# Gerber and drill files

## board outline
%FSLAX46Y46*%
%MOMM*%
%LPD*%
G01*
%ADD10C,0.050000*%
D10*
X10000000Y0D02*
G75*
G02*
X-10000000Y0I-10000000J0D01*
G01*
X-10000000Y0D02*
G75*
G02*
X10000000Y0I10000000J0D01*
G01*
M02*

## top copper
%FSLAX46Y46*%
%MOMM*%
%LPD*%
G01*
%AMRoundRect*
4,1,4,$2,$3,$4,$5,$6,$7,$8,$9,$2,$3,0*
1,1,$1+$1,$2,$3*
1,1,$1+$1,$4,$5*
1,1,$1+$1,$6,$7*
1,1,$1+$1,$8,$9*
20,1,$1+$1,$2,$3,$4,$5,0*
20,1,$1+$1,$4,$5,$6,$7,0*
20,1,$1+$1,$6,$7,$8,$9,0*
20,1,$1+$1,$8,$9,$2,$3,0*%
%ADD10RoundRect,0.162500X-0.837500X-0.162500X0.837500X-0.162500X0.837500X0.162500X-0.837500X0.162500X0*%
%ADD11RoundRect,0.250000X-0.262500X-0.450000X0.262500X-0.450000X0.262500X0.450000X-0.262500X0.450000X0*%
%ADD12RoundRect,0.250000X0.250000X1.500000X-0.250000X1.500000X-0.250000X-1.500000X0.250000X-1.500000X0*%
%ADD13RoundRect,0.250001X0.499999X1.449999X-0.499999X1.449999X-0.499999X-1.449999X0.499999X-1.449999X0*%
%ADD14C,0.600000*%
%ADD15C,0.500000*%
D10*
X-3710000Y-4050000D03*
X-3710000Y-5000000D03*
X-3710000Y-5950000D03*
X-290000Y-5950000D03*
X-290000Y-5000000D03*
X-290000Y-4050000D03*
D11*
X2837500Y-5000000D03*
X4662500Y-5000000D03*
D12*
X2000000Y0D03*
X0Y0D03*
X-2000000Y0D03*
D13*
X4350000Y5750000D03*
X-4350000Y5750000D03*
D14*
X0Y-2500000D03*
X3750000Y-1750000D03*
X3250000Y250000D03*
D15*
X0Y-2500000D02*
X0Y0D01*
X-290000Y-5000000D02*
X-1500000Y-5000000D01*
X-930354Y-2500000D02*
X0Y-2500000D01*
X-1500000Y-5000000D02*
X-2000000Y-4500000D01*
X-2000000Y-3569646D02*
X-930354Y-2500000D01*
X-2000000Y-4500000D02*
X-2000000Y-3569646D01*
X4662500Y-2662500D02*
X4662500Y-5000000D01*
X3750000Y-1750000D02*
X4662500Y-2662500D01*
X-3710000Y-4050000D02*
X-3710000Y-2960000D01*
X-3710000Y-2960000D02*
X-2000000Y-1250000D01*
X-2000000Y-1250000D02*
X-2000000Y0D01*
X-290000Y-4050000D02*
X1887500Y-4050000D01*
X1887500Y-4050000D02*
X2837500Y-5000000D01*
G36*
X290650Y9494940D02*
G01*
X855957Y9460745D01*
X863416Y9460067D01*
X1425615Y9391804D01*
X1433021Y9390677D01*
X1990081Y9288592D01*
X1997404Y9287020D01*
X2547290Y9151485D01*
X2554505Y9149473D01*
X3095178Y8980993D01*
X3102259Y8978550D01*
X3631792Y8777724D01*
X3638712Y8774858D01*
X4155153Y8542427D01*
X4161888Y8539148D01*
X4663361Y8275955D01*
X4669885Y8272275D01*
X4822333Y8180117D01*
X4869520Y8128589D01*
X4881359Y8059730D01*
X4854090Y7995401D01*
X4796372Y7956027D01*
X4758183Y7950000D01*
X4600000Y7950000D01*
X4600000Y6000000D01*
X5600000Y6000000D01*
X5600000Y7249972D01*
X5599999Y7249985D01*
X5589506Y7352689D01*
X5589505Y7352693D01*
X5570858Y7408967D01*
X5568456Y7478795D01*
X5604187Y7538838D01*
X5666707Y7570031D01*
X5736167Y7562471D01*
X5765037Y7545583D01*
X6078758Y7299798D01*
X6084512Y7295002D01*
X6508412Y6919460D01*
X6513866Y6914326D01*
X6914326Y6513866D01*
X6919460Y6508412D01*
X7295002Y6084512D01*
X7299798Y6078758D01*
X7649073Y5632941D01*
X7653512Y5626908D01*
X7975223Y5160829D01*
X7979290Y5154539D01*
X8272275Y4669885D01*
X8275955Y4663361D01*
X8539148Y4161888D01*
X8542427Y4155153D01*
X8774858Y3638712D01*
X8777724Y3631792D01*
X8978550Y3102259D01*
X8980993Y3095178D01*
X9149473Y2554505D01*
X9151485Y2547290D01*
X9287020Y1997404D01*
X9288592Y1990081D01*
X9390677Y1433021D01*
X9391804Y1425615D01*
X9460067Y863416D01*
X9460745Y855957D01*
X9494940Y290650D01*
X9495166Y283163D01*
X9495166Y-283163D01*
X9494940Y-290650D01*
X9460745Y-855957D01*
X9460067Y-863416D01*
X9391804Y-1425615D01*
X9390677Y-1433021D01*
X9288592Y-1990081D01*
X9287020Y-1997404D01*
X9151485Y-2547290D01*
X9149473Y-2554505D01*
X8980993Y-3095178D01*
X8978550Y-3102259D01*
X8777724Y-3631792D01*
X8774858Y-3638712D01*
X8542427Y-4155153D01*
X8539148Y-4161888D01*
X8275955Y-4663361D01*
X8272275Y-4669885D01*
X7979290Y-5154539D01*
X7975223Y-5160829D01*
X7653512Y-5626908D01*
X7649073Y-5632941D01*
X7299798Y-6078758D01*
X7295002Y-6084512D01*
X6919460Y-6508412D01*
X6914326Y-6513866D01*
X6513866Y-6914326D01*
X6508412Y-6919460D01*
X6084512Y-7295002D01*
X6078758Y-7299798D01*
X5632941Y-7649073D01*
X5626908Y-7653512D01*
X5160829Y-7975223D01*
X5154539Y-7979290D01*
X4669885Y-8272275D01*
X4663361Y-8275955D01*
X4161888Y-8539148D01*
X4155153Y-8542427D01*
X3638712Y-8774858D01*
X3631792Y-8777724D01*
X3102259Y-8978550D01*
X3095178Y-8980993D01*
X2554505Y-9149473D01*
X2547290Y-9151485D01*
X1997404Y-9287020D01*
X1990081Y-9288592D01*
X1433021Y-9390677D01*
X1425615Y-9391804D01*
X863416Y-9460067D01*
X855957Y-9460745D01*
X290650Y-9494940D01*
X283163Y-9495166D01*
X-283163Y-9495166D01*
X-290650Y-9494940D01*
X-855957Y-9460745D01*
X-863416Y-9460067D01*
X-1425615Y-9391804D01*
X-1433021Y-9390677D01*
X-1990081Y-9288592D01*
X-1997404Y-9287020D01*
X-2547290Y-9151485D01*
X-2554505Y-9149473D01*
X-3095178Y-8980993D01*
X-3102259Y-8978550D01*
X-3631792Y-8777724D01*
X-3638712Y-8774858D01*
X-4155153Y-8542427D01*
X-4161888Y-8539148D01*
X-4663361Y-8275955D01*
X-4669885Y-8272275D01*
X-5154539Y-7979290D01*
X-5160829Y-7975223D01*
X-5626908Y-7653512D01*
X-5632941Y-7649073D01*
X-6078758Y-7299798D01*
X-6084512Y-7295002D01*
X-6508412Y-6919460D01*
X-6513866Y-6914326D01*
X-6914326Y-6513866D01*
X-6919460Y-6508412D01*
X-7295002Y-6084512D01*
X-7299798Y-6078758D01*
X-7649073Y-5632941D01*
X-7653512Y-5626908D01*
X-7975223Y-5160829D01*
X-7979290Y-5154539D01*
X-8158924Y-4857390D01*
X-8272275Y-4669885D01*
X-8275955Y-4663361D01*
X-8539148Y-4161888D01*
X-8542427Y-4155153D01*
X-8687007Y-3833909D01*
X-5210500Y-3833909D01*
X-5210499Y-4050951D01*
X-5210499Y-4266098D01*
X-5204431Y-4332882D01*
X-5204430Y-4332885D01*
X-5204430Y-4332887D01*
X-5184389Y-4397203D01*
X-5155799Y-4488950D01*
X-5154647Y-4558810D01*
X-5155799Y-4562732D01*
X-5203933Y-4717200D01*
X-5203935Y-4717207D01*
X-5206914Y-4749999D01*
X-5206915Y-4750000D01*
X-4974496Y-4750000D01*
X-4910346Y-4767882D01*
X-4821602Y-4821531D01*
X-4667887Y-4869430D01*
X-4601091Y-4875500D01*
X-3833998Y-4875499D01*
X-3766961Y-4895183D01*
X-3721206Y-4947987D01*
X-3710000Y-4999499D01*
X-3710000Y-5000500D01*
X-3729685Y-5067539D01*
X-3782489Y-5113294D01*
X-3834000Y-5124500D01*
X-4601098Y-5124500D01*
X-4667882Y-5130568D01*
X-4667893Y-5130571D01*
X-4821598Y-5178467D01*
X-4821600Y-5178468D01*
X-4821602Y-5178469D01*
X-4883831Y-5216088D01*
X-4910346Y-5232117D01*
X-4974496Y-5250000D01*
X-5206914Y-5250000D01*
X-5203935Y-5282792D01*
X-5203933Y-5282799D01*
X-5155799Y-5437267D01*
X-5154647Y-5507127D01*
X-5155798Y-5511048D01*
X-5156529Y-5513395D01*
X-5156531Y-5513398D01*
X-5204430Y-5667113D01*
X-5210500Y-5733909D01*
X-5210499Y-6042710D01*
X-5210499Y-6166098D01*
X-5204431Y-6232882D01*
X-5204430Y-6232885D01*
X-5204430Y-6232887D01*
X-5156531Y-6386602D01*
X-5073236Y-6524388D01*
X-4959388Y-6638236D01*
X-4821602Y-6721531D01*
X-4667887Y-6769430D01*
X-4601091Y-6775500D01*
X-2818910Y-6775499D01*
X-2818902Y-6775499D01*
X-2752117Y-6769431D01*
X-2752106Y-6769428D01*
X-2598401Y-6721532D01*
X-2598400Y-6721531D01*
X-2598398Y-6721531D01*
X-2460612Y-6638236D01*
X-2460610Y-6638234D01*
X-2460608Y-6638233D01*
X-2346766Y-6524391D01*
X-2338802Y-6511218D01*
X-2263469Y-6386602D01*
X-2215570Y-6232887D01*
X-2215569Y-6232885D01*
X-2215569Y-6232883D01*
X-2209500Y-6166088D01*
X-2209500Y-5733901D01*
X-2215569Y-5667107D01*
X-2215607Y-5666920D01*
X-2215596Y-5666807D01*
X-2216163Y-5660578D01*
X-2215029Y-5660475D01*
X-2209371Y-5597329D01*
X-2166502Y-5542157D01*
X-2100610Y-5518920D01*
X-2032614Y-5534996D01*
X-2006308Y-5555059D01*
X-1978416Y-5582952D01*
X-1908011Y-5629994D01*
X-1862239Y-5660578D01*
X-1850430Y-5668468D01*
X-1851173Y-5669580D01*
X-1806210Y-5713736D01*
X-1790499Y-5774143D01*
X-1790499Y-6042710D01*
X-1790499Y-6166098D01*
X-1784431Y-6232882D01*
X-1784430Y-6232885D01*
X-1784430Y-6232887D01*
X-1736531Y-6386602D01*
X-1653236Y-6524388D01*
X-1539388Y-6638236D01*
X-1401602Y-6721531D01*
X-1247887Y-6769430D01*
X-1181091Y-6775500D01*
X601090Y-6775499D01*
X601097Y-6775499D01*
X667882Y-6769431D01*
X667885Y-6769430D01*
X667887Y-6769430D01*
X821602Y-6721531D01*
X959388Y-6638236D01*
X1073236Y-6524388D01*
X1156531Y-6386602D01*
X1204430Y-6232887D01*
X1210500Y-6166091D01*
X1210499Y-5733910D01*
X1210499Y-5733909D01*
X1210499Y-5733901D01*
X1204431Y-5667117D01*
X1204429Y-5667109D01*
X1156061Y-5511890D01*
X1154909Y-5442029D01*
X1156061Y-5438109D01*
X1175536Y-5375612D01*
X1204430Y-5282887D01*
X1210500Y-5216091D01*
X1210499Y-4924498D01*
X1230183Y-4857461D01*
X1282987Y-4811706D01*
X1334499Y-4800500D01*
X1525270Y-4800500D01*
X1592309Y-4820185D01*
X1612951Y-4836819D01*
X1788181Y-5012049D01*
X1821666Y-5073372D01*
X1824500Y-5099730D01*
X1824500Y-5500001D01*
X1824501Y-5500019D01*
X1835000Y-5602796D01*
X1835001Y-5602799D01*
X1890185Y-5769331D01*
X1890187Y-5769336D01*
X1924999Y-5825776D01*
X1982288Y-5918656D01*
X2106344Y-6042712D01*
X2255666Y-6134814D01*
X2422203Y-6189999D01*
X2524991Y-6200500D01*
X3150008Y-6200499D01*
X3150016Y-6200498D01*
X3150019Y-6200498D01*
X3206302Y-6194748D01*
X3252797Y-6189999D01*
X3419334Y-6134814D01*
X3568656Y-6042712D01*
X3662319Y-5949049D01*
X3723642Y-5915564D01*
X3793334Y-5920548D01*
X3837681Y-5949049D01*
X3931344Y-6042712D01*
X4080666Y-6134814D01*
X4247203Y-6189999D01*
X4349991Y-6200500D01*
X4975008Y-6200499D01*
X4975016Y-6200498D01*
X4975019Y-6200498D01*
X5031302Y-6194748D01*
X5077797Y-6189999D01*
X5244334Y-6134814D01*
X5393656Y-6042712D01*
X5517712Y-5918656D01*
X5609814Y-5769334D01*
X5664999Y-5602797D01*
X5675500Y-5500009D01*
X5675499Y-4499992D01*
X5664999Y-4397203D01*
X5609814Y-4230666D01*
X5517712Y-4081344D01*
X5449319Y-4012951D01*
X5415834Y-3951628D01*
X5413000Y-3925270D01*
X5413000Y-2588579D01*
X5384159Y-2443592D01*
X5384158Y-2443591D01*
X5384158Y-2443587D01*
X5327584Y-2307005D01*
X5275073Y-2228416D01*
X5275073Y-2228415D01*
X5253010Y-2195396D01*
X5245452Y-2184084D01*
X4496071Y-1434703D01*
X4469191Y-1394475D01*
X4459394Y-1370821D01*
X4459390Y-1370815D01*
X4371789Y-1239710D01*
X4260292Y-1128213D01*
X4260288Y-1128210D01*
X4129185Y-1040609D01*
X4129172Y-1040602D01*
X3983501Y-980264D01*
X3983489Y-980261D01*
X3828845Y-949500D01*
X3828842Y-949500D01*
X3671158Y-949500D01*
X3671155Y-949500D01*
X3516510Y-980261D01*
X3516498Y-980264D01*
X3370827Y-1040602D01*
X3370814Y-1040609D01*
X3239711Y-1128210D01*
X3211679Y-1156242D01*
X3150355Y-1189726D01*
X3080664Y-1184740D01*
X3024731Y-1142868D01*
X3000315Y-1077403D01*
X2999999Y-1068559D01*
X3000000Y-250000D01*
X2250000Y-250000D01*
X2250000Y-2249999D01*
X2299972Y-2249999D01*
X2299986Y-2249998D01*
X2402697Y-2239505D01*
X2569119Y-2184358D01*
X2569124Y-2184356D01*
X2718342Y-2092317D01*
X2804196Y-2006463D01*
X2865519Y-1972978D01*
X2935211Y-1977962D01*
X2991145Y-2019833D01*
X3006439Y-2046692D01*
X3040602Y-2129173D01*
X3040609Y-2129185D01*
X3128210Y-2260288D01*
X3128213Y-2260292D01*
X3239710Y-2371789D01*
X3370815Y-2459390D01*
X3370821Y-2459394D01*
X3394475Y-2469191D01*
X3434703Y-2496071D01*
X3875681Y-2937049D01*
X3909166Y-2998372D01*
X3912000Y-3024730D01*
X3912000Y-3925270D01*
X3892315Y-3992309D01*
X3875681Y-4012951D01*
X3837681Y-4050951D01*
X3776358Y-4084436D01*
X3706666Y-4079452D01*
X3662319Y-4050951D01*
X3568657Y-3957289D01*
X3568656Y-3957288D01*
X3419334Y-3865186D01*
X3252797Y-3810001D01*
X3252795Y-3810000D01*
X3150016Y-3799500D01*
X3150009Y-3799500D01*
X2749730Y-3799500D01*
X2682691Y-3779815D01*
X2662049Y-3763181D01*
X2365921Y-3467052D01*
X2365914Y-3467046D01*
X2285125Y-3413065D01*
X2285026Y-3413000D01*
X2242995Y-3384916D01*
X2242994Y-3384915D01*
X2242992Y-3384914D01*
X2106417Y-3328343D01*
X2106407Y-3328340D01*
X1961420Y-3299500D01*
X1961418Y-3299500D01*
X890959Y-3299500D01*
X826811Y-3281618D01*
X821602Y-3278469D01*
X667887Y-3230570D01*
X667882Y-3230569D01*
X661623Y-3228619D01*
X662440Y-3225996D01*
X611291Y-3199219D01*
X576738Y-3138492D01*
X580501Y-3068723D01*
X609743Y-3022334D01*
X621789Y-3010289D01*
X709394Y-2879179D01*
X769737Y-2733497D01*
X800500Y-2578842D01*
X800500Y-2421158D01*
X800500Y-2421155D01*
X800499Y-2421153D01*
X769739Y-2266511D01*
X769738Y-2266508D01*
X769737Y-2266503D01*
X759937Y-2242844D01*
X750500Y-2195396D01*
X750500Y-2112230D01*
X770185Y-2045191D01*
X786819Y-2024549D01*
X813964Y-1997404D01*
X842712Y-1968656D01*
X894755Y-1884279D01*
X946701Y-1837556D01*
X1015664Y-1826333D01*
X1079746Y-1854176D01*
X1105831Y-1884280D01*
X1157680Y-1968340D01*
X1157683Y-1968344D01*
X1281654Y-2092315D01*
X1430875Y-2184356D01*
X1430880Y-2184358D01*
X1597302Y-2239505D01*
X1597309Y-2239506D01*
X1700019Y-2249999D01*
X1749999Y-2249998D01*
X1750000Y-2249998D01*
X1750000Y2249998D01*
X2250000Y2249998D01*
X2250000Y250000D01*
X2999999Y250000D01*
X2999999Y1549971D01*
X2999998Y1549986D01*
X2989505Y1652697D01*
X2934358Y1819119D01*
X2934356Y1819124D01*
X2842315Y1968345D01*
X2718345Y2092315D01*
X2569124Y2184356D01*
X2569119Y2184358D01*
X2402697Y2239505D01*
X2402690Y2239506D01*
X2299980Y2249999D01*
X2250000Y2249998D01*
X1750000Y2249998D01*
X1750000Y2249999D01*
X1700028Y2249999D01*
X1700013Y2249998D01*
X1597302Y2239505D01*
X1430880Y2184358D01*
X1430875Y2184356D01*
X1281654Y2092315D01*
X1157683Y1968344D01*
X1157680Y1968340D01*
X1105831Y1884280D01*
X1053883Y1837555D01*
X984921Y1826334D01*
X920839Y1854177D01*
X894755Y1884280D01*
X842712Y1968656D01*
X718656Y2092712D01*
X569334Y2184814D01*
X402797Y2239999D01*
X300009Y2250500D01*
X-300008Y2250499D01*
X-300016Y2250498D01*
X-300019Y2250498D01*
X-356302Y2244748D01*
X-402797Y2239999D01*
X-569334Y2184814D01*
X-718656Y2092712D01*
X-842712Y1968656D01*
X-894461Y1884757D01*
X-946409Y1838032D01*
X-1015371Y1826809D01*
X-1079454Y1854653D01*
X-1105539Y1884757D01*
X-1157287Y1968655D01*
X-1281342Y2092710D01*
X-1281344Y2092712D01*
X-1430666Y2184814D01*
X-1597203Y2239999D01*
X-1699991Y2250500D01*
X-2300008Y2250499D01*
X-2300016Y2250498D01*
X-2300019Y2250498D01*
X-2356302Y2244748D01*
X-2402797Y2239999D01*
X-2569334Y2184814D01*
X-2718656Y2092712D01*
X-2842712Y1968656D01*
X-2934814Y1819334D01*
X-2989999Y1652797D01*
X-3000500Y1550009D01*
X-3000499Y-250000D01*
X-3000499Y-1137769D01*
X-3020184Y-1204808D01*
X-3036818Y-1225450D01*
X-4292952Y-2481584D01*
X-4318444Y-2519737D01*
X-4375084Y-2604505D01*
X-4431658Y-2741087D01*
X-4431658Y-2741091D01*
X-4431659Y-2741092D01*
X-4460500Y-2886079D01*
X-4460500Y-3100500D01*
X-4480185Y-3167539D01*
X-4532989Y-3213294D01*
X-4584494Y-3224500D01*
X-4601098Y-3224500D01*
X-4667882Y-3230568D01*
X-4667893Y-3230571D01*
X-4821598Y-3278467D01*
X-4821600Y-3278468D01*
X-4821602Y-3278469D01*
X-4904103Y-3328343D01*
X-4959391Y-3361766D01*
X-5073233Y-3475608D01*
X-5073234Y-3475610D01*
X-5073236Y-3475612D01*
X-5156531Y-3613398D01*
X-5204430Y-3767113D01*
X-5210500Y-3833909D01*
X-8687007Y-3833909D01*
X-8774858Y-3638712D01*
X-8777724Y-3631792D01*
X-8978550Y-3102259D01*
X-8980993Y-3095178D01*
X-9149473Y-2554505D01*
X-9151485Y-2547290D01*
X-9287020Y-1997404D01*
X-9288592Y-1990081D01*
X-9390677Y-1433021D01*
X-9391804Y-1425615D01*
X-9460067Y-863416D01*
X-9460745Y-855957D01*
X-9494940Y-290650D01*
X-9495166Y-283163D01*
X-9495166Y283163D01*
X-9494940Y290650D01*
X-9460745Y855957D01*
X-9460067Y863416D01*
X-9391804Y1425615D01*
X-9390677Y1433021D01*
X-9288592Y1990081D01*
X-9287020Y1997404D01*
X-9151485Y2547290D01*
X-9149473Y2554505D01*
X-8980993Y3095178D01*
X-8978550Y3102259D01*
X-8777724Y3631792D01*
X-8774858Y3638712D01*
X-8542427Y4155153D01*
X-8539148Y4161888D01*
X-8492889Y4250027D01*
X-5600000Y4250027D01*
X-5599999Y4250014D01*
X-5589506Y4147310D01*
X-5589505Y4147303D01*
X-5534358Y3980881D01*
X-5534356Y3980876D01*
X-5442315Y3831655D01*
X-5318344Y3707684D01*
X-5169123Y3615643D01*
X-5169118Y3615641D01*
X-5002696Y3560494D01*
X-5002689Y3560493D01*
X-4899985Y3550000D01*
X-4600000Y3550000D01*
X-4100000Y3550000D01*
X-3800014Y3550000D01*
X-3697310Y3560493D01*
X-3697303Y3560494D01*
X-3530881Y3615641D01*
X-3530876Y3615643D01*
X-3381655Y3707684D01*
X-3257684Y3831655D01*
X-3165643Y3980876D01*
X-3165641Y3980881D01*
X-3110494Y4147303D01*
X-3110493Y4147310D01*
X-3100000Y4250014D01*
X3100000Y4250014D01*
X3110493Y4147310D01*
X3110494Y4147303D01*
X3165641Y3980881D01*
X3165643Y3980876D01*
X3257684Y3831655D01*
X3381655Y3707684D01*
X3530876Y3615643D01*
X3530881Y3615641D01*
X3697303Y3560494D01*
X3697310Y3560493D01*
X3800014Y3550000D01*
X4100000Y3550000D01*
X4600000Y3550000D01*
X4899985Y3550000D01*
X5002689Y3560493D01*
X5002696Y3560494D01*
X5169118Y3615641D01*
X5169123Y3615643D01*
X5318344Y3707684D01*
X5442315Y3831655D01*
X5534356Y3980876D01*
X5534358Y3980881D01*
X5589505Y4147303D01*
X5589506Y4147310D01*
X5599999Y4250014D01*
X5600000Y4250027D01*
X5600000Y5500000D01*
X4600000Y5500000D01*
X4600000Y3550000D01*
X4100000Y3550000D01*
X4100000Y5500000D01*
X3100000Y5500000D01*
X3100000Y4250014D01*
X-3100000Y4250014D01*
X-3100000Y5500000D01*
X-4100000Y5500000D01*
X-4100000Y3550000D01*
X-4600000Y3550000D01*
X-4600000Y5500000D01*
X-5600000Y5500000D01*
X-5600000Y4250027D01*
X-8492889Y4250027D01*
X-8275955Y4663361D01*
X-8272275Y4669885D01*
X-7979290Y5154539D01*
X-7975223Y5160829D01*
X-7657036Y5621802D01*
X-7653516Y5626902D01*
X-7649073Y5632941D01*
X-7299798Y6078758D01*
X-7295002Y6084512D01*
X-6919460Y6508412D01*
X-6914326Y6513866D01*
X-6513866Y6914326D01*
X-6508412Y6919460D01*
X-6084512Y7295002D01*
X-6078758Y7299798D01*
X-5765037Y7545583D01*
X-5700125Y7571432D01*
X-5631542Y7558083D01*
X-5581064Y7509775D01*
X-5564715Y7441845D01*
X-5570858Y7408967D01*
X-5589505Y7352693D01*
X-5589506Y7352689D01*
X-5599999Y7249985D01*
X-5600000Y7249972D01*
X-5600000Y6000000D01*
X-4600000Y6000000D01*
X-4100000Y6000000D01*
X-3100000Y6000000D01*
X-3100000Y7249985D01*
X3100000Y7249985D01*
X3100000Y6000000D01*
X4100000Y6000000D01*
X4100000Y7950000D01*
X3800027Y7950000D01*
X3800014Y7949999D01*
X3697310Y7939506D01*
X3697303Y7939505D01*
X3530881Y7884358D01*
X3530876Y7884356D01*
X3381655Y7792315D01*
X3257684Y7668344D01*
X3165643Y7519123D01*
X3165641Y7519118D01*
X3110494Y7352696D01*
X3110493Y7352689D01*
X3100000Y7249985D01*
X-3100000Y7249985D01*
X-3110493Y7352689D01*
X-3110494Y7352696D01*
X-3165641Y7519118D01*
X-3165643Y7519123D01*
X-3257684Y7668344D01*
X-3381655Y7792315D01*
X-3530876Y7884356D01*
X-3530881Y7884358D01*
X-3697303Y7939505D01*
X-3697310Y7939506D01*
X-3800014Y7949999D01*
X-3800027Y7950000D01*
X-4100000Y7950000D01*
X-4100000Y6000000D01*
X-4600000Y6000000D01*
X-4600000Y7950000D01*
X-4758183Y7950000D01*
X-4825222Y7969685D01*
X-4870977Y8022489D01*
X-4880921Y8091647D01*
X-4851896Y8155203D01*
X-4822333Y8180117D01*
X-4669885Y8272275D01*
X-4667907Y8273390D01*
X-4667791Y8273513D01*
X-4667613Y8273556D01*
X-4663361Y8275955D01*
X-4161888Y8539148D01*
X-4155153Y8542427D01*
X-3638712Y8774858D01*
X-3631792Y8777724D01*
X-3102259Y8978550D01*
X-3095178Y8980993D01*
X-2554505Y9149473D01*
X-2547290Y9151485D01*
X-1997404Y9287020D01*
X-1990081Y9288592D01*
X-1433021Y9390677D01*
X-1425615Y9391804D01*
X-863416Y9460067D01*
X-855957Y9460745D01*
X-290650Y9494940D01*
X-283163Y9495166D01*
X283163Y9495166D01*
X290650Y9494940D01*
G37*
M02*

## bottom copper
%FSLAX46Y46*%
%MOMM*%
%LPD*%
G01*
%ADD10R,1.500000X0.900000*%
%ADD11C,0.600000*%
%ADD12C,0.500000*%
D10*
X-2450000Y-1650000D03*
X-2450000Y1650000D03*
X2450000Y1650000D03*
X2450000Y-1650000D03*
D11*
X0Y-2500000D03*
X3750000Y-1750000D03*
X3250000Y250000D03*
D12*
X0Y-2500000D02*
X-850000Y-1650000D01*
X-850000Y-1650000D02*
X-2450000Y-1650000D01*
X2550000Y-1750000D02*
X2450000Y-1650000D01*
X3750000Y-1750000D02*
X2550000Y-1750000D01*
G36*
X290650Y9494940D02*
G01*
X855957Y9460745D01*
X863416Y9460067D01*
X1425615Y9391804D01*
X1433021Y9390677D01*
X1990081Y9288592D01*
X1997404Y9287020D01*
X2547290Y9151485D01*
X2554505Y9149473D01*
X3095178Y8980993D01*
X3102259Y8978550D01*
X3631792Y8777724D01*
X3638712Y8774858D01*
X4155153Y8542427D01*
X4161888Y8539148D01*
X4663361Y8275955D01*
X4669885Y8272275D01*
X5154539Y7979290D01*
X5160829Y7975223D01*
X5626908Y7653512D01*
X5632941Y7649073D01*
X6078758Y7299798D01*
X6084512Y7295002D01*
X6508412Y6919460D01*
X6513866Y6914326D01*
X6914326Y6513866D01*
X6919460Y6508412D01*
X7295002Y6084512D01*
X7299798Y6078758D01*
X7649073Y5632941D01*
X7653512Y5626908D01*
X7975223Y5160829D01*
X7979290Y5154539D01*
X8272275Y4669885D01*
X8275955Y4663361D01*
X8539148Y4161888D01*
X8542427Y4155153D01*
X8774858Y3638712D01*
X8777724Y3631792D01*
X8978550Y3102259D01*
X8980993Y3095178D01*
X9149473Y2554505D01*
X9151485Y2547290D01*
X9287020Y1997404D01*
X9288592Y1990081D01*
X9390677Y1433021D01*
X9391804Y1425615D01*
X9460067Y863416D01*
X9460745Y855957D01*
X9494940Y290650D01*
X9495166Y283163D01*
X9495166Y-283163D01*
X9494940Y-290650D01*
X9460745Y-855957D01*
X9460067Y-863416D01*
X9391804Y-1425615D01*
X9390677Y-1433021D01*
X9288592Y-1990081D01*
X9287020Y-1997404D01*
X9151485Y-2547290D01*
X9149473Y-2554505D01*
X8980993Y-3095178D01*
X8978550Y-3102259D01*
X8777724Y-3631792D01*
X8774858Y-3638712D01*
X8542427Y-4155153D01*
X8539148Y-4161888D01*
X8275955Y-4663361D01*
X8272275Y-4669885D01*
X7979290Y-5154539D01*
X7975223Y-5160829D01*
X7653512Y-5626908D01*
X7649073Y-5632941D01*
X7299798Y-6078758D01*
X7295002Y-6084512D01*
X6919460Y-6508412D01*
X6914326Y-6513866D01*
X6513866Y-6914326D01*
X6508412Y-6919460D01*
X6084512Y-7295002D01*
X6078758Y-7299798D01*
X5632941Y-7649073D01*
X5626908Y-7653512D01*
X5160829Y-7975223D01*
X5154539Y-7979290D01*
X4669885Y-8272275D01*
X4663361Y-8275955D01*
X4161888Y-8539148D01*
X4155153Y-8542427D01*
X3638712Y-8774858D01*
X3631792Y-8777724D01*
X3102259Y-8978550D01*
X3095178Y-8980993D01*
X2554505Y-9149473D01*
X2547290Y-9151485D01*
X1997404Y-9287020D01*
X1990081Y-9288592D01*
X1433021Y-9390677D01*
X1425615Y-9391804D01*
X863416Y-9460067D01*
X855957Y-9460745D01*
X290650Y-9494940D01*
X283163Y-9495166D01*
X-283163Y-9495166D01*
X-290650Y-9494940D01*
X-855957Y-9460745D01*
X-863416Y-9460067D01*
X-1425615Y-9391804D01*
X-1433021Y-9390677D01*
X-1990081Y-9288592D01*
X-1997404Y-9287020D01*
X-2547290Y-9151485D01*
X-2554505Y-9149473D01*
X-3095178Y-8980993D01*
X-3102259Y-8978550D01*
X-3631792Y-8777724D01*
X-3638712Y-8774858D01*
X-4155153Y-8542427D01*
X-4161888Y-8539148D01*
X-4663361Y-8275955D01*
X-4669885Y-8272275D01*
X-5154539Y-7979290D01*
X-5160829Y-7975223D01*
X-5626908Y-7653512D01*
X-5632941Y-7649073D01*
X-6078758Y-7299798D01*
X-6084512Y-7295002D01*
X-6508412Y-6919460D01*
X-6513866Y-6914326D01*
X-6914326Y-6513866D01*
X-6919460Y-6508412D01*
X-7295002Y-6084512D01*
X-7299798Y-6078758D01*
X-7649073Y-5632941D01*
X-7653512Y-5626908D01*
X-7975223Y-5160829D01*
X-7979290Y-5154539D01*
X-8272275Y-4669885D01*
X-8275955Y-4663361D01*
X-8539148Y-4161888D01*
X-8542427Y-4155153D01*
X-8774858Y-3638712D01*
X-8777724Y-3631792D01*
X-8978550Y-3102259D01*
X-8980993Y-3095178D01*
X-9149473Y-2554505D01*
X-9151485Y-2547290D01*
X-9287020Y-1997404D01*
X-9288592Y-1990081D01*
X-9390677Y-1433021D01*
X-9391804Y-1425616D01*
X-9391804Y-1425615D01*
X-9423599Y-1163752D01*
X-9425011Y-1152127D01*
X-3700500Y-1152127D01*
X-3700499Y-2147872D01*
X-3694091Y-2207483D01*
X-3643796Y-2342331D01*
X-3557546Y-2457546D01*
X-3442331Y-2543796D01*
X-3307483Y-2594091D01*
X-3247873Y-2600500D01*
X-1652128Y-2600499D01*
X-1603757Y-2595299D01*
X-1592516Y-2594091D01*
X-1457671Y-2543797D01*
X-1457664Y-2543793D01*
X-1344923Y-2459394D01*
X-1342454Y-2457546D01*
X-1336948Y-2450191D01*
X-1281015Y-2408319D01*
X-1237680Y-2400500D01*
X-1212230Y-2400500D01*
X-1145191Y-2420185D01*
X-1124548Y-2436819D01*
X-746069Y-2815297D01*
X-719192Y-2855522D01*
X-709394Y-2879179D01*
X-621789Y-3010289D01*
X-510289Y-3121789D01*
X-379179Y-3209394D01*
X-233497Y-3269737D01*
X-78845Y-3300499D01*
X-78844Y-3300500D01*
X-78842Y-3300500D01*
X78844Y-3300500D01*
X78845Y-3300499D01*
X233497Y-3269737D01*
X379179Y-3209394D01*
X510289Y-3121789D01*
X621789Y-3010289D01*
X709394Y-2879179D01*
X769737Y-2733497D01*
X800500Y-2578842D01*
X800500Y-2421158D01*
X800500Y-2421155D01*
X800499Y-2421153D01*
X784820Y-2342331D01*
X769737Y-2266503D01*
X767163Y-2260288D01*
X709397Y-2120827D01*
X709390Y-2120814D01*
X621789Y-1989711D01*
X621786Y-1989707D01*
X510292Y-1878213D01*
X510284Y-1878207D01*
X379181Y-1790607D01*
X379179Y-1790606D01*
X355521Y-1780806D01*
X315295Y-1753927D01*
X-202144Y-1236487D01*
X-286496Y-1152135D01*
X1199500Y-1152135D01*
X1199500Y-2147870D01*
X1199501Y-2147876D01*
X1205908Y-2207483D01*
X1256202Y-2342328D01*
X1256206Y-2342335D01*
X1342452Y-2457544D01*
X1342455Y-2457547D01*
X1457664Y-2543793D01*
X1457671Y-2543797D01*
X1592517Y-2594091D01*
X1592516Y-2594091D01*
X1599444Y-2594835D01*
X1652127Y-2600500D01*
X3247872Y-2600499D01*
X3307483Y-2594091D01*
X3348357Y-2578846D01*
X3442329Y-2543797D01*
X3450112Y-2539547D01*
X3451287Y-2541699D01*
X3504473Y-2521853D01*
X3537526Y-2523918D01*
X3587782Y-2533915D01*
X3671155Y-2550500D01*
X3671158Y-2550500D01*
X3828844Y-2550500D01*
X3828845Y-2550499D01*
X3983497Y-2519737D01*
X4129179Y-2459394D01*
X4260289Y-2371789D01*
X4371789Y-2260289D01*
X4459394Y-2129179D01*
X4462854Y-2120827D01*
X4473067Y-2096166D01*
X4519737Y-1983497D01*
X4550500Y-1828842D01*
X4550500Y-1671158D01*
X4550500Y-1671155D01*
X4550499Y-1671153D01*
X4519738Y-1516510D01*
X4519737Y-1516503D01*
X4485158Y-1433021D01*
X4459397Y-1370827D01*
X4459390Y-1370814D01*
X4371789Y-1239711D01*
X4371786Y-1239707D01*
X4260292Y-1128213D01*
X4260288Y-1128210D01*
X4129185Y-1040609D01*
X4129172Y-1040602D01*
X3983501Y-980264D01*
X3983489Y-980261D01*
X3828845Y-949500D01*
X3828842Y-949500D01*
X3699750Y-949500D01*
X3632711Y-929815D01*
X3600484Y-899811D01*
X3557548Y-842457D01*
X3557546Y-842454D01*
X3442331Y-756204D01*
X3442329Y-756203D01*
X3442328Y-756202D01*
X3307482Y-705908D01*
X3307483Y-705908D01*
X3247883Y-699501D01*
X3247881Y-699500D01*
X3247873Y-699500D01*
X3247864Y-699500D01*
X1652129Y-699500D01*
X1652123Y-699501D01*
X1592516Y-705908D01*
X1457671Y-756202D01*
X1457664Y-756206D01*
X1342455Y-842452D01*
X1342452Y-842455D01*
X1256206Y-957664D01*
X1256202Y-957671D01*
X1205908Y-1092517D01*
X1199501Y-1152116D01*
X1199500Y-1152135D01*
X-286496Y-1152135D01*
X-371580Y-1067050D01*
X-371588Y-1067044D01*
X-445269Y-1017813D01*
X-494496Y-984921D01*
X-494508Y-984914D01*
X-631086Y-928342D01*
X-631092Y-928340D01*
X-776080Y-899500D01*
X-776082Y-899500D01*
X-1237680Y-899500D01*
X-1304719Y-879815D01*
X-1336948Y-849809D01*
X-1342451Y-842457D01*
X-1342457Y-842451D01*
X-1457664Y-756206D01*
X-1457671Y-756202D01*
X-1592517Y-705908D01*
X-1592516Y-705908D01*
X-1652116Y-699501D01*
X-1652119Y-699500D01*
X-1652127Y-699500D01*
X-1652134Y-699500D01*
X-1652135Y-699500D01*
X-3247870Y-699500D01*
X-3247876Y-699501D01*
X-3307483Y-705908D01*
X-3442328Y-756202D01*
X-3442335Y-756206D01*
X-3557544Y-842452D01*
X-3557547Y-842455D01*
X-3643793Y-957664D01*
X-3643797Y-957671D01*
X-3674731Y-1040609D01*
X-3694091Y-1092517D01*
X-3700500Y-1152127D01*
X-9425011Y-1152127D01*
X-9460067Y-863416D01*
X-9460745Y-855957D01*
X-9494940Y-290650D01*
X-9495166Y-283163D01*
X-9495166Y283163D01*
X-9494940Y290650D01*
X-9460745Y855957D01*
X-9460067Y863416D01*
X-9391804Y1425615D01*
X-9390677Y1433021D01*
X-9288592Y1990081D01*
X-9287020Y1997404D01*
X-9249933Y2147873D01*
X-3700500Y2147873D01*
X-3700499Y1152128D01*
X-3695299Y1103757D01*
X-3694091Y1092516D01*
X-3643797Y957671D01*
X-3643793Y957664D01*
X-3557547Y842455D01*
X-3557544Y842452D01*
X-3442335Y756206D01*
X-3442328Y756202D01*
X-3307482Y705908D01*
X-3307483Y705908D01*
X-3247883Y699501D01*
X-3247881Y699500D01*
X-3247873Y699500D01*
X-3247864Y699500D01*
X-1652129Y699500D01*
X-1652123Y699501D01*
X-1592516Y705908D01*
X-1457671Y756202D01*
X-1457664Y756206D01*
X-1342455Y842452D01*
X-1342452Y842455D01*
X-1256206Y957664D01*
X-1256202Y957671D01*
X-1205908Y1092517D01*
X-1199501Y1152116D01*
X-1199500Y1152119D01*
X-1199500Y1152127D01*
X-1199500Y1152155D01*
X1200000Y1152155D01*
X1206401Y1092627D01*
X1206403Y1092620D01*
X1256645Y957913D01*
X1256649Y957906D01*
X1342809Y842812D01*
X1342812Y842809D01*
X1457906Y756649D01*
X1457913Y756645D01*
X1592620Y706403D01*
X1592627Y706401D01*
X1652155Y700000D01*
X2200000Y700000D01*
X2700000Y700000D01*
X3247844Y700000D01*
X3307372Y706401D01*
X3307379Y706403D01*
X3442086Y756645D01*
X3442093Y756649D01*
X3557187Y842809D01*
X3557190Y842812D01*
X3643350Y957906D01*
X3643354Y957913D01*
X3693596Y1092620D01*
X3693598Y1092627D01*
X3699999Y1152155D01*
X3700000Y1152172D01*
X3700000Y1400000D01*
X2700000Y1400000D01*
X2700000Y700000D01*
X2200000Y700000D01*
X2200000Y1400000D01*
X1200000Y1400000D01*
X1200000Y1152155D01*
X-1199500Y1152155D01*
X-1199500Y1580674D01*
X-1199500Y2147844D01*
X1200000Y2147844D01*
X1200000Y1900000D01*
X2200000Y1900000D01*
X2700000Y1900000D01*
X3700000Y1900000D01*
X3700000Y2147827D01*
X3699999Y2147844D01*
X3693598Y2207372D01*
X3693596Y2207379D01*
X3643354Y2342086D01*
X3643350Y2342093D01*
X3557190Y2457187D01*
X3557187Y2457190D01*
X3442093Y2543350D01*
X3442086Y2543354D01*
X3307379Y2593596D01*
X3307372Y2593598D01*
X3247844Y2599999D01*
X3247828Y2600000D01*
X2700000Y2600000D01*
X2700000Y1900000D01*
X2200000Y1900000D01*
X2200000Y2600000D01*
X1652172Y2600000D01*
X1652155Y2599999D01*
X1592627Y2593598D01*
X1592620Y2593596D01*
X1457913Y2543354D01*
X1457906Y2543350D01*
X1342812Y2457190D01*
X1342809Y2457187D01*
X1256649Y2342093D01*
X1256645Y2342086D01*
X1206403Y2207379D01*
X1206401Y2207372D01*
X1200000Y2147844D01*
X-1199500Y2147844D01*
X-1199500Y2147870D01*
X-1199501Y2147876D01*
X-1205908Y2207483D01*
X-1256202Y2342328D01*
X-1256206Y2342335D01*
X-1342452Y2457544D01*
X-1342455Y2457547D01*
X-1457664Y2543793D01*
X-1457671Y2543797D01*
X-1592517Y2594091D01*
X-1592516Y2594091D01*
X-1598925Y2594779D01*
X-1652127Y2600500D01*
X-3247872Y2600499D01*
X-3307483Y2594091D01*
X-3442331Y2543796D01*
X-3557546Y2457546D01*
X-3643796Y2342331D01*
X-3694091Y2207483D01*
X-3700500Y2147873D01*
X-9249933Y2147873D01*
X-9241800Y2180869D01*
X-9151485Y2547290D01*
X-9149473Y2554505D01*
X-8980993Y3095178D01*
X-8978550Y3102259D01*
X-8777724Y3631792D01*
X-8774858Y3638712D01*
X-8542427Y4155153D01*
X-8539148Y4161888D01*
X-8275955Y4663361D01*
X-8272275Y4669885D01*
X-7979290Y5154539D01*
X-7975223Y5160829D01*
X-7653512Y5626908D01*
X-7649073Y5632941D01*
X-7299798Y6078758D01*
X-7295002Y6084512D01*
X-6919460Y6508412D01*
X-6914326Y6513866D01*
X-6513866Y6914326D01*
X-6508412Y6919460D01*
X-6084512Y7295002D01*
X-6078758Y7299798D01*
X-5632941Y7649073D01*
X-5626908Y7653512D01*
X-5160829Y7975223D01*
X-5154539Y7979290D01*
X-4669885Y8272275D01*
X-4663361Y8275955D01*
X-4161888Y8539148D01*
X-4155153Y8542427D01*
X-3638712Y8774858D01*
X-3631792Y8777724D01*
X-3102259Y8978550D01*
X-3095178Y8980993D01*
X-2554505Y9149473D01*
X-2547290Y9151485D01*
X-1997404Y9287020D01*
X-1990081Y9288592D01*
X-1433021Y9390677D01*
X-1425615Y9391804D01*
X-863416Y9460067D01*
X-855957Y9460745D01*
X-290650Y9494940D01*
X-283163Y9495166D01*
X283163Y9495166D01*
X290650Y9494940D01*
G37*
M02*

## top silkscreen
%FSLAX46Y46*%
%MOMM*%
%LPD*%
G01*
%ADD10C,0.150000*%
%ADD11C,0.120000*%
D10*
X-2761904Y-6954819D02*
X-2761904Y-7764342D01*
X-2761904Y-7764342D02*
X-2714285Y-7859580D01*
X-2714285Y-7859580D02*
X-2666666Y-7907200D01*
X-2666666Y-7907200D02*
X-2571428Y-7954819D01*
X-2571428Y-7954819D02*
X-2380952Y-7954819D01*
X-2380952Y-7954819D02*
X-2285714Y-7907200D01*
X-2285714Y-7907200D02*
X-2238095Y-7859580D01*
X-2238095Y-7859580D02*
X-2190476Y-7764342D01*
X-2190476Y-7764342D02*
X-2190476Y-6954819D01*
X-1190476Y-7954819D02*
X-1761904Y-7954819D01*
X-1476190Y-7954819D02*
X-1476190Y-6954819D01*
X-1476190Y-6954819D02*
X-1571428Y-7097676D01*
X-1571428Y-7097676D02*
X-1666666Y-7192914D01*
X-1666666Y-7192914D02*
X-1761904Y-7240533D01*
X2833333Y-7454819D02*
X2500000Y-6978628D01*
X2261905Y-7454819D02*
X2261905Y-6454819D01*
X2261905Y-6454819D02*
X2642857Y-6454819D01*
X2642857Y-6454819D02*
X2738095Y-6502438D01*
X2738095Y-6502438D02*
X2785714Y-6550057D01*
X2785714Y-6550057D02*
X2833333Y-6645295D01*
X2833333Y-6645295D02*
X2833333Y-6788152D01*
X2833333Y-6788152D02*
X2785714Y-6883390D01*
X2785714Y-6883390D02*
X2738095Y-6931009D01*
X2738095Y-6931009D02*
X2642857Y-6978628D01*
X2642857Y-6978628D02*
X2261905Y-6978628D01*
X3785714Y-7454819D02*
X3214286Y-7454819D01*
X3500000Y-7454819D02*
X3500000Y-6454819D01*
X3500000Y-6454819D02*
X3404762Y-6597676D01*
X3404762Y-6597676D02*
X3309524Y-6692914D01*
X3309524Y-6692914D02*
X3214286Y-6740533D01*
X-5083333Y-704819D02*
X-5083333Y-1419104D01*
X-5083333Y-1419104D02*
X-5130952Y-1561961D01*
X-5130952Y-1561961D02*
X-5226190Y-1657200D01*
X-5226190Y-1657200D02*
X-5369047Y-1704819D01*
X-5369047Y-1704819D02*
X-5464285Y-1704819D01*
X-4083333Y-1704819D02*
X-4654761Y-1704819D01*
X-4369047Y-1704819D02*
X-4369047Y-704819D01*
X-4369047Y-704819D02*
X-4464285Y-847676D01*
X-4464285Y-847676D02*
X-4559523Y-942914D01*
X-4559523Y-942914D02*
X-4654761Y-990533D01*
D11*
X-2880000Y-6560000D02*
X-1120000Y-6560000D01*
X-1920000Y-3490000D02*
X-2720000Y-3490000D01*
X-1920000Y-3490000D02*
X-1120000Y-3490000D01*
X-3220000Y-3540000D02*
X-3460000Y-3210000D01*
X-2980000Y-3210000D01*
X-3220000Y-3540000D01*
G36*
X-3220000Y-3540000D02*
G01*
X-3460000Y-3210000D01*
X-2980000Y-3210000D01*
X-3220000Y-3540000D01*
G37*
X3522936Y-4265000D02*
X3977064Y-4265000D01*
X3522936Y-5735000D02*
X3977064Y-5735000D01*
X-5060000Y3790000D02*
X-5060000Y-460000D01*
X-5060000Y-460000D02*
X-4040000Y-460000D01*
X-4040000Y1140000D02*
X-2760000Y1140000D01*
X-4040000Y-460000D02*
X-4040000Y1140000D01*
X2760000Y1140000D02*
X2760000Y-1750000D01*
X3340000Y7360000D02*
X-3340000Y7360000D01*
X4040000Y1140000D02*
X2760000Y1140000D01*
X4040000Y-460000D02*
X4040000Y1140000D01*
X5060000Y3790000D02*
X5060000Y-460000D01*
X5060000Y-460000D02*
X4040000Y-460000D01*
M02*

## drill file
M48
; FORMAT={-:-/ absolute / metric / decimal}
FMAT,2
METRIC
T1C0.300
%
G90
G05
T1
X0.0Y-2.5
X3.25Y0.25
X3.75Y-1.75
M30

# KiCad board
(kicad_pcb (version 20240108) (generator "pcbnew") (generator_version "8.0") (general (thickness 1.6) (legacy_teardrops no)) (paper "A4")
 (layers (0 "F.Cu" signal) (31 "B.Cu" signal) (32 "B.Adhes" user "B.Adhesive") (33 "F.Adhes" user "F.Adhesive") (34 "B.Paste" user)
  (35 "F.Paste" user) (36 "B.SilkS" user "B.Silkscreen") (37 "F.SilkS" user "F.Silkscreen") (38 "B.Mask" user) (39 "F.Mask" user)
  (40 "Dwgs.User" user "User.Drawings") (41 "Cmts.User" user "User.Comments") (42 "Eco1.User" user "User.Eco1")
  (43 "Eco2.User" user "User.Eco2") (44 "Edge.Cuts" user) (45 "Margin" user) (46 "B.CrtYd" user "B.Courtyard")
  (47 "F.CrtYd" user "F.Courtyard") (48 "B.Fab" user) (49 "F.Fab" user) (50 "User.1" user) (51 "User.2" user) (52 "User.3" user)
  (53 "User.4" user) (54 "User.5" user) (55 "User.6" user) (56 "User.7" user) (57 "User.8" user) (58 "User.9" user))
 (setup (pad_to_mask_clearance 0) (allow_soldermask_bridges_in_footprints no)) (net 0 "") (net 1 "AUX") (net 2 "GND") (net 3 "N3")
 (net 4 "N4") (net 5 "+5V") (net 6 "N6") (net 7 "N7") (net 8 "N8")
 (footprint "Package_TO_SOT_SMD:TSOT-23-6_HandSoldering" (layer "F.Cu") (at -2 5)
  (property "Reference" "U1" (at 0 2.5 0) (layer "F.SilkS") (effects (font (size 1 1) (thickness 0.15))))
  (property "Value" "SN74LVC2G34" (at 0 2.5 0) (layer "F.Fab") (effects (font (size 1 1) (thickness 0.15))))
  (fp_line (start -0.88 1.56) (end 0.88 1.56) (stroke (width 0.12) (type solid)) (layer "F.SilkS"))
  (fp_line (start 0.08 -1.51) (end -0.72 -1.51) (stroke (width 0.12) (type solid)) (layer "F.SilkS"))
  (fp_line (start 0.08 -1.51) (end 0.88 -1.51) (stroke (width 0.12) (type solid)) (layer "F.SilkS"))
  (fp_poly
   (pts (xy -1.22 -1.46) (xy -1.46 -1.79) (xy -0.98 -1.79) (xy -1.22 -1.46)) (stroke (width 0.12) (type solid)) (fill solid)
   (layer "F.SilkS"))
  (pad "1" smd roundrect (at -1.71 -0.95) (size 2 0.65) (layers "F.Cu" "F.Paste" "F.Mask") (roundrect_rratio 0.25) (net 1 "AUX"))
  (pad "2" smd roundrect (at -1.71 0) (size 2 0.65) (layers "F.Cu" "F.Paste" "F.Mask") (roundrect_rratio 0.25) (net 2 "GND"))
  (pad "3" smd roundrect (at -1.71 0.95) (size 2 0.65) (layers "F.Cu" "F.Paste" "F.Mask") (roundrect_rratio 0.25) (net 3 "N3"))
  (pad "4" smd roundrect (at 1.71 0.95) (size 2 0.65) (layers "F.Cu" "F.Paste" "F.Mask") (roundrect_rratio 0.25) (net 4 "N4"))
  (pad "5" smd roundrect (at 1.71 0) (size 2 0.65) (layers "F.Cu" "F.Paste" "F.Mask") (roundrect_rratio 0.25) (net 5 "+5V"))
  (pad "6" smd roundrect (at 1.71 -0.95) (size 2 0.65) (layers "F.Cu" "F.Paste" "F.Mask") (roundrect_rratio 0.25) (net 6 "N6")))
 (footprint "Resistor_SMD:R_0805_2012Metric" (layer "F.Cu") (at 3.75 5)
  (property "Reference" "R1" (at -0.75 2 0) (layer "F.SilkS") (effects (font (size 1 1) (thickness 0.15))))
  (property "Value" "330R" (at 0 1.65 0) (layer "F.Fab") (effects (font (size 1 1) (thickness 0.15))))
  (fp_line (start -0.227064 -0.735) (end 0.227064 -0.735) (stroke (width 0.12) (type solid)) (layer "F.SilkS"))
  (fp_line (start -0.227064 0.735) (end 0.227064 0.735) (stroke (width 0.12) (type solid)) (layer "F.SilkS"))
  (pad "1" smd roundrect (at -0.9125 0) (size 1.025 1.4) (layers "F.Cu" "F.Paste" "F.Mask") (roundrect_rratio 0.243902) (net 6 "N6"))
  (pad "2" smd roundrect (at 0.9125 0) (size 1.025 1.4) (layers "F.Cu" "F.Paste" "F.Mask") (roundrect_rratio 0.243902) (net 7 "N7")))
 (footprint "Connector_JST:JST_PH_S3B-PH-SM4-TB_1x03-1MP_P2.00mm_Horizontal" (layer "F.Cu") (at 0 -2.85 180)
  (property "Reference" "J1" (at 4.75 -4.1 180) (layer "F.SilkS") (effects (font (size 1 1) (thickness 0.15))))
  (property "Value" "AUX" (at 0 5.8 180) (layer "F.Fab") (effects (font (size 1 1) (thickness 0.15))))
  (fp_line (start 5.06 0.94) (end 5.06 -3.31) (stroke (width 0.12) (type solid)) (layer "F.SilkS"))
  (fp_line (start 5.06 -3.31) (end 4.04 -3.31) (stroke (width 0.12) (type solid)) (layer "F.SilkS"))
  (fp_line (start 4.04 -1.71) (end 2.76 -1.71) (stroke (width 0.12) (type solid)) (layer "F.SilkS"))
  (fp_line (start 4.04 -3.31) (end 4.04 -1.71) (stroke (width 0.12) (type solid)) (layer "F.SilkS"))
  (fp_line (start -2.76 -1.71) (end -2.76 -4.6) (stroke (width 0.12) (type solid)) (layer "F.SilkS"))
  (fp_line (start -3.34 4.51) (end 3.34 4.51) (stroke (width 0.12) (type solid)) (layer "F.SilkS"))
  (fp_line (start -4.04 -1.71) (end -2.76 -1.71) (stroke (width 0.12) (type solid)) (layer "F.SilkS"))
  (fp_line (start -4.04 -3.31) (end -4.04 -1.71) (stroke (width 0.12) (type solid)) (layer "F.SilkS"))
  (fp_line (start -5.06 0.94) (end -5.06 -3.31) (stroke (width 0.12) (type solid)) (layer "F.SilkS"))
  (fp_line (start -5.06 -3.31) (end -4.04 -3.31) (stroke (width 0.12) (type solid)) (layer "F.SilkS"))
  (pad "1" smd roundrect (at -2 -2.85 180) (size 1 3.5) (layers "F.Cu" "F.Paste" "F.Mask") (roundrect_rratio 0.25) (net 2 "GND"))
  (pad "2" smd roundrect (at 0 -2.85 180) (size 1 3.5) (layers "F.Cu" "F.Paste" "F.Mask") (roundrect_rratio 0.25) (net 5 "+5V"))
  (pad "3" smd roundrect (at 2 -2.85 180) (size 1 3.5) (layers "F.Cu" "F.Paste" "F.Mask") (roundrect_rratio 0.25) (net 1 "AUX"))
  (pad "MP" smd roundrect (at -4.35 2.9 180) (size 1.5 3.4) (layers "F.Cu" "F.Paste" "F.Mask") (roundrect_rratio 0.166667) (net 2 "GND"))
  (pad "MP" smd roundrect (at 4.35 2.9 180) (size 1.5 3.4) (layers "F.Cu" "F.Paste" "F.Mask") (roundrect_rratio 0.166667) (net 2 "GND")))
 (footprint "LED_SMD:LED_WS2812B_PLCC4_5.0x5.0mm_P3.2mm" (layer "B.Cu") (at 0 0)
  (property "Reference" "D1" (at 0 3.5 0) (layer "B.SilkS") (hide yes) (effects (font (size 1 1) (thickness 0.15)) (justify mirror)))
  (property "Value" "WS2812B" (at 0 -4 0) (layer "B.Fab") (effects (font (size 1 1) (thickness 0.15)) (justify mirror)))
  (pad "1" smd rect (at -2.45 1.65) (size 1.5 0.9) (layers "B.Cu" "B.Paste" "B.Mask") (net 5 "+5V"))
  (pad "2" smd rect (at -2.45 -1.65) (size 1.5 0.9) (layers "B.Cu" "B.Paste" "B.Mask") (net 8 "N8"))
  (pad "3" smd rect (at 2.45 -1.65) (size 1.5 0.9) (layers "B.Cu" "B.Paste" "B.Mask") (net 2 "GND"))
  (pad "4" smd rect (at 2.45 1.65) (size 1.5 0.9) (layers "B.Cu" "B.Paste" "B.Mask") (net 7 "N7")))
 (gr_circle (center 0 0) (end 10 0) (stroke (width 0.05) (type default)) (fill none) (layer "Edge.Cuts"))
 (segment (start 0 2.5) (end 0 0) (width 0.5) (layer "F.Cu") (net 5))
 (segment (start -0.29 5) (end -1.5 5) (width 0.5) (layer "F.Cu") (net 5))
 (segment (start -0.930354 2.5) (end 0 2.5) (width 0.5) (layer "F.Cu") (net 5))
 (segment (start -1.5 5) (end -2 4.5) (width 0.5) (layer "F.Cu") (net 5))
 (segment (start -2 3.569646) (end -0.930354 2.5) (width 0.5) (layer "F.Cu") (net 5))
 (segment (start -2 4.5) (end -2 3.569646) (width 0.5) (layer "F.Cu") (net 5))
 (via (at 0 2.5) (size 0.6) (drill 0.3) (layers "F.Cu" "B.Cu") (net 5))
 (segment (start 0 2.5) (end -0.85 1.65) (width 0.5) (layer "B.Cu") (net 5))
 (segment (start -0.85 1.65) (end -2.45 1.65) (width 0.5) (layer "B.Cu") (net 5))
 (segment (start 4.6625 2.6625) (end 4.6625 5) (width 0.5) (layer "F.Cu") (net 7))
 (segment (start 3.75 1.75) (end 4.6625 2.6625) (width 0.5) (layer "F.Cu") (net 7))
 (via (at 3.75 1.75) (size 0.6) (drill 0.3) (layers "F.Cu" "B.Cu") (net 7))
 (segment (start 2.55 1.75) (end 2.45 1.65) (width 0.5) (layer "B.Cu") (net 7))
 (segment (start 3.75 1.75) (end 2.55 1.75) (width 0.5) (layer "B.Cu") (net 7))
 (via (at 3.25 -0.25) (size 0.6) (drill 0.3) (layers "F.Cu" "B.Cu") (free yes) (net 2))
 (segment (start -3.71 4.05) (end -3.71 2.96) (width 0.5) (layer "F.Cu") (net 1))
 (segment (start -3.71 2.96) (end -2 1.25) (width 0.5) (layer "F.Cu") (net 1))
 (segment (start -2 1.25) (end -2 0) (width 0.5) (layer "F.Cu") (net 1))
 (segment (start -0.29 4.05) (end 1.8875 4.05) (width 0.5) (layer "F.Cu") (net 6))
 (segment (start 1.8875 4.05) (end 2.8375 5) (width 0.5) (layer "F.Cu") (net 6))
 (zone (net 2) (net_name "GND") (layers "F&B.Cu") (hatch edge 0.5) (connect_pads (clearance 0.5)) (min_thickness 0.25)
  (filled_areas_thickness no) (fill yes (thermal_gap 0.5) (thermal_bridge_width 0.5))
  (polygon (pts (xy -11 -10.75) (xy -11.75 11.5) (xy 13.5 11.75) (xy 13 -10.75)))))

